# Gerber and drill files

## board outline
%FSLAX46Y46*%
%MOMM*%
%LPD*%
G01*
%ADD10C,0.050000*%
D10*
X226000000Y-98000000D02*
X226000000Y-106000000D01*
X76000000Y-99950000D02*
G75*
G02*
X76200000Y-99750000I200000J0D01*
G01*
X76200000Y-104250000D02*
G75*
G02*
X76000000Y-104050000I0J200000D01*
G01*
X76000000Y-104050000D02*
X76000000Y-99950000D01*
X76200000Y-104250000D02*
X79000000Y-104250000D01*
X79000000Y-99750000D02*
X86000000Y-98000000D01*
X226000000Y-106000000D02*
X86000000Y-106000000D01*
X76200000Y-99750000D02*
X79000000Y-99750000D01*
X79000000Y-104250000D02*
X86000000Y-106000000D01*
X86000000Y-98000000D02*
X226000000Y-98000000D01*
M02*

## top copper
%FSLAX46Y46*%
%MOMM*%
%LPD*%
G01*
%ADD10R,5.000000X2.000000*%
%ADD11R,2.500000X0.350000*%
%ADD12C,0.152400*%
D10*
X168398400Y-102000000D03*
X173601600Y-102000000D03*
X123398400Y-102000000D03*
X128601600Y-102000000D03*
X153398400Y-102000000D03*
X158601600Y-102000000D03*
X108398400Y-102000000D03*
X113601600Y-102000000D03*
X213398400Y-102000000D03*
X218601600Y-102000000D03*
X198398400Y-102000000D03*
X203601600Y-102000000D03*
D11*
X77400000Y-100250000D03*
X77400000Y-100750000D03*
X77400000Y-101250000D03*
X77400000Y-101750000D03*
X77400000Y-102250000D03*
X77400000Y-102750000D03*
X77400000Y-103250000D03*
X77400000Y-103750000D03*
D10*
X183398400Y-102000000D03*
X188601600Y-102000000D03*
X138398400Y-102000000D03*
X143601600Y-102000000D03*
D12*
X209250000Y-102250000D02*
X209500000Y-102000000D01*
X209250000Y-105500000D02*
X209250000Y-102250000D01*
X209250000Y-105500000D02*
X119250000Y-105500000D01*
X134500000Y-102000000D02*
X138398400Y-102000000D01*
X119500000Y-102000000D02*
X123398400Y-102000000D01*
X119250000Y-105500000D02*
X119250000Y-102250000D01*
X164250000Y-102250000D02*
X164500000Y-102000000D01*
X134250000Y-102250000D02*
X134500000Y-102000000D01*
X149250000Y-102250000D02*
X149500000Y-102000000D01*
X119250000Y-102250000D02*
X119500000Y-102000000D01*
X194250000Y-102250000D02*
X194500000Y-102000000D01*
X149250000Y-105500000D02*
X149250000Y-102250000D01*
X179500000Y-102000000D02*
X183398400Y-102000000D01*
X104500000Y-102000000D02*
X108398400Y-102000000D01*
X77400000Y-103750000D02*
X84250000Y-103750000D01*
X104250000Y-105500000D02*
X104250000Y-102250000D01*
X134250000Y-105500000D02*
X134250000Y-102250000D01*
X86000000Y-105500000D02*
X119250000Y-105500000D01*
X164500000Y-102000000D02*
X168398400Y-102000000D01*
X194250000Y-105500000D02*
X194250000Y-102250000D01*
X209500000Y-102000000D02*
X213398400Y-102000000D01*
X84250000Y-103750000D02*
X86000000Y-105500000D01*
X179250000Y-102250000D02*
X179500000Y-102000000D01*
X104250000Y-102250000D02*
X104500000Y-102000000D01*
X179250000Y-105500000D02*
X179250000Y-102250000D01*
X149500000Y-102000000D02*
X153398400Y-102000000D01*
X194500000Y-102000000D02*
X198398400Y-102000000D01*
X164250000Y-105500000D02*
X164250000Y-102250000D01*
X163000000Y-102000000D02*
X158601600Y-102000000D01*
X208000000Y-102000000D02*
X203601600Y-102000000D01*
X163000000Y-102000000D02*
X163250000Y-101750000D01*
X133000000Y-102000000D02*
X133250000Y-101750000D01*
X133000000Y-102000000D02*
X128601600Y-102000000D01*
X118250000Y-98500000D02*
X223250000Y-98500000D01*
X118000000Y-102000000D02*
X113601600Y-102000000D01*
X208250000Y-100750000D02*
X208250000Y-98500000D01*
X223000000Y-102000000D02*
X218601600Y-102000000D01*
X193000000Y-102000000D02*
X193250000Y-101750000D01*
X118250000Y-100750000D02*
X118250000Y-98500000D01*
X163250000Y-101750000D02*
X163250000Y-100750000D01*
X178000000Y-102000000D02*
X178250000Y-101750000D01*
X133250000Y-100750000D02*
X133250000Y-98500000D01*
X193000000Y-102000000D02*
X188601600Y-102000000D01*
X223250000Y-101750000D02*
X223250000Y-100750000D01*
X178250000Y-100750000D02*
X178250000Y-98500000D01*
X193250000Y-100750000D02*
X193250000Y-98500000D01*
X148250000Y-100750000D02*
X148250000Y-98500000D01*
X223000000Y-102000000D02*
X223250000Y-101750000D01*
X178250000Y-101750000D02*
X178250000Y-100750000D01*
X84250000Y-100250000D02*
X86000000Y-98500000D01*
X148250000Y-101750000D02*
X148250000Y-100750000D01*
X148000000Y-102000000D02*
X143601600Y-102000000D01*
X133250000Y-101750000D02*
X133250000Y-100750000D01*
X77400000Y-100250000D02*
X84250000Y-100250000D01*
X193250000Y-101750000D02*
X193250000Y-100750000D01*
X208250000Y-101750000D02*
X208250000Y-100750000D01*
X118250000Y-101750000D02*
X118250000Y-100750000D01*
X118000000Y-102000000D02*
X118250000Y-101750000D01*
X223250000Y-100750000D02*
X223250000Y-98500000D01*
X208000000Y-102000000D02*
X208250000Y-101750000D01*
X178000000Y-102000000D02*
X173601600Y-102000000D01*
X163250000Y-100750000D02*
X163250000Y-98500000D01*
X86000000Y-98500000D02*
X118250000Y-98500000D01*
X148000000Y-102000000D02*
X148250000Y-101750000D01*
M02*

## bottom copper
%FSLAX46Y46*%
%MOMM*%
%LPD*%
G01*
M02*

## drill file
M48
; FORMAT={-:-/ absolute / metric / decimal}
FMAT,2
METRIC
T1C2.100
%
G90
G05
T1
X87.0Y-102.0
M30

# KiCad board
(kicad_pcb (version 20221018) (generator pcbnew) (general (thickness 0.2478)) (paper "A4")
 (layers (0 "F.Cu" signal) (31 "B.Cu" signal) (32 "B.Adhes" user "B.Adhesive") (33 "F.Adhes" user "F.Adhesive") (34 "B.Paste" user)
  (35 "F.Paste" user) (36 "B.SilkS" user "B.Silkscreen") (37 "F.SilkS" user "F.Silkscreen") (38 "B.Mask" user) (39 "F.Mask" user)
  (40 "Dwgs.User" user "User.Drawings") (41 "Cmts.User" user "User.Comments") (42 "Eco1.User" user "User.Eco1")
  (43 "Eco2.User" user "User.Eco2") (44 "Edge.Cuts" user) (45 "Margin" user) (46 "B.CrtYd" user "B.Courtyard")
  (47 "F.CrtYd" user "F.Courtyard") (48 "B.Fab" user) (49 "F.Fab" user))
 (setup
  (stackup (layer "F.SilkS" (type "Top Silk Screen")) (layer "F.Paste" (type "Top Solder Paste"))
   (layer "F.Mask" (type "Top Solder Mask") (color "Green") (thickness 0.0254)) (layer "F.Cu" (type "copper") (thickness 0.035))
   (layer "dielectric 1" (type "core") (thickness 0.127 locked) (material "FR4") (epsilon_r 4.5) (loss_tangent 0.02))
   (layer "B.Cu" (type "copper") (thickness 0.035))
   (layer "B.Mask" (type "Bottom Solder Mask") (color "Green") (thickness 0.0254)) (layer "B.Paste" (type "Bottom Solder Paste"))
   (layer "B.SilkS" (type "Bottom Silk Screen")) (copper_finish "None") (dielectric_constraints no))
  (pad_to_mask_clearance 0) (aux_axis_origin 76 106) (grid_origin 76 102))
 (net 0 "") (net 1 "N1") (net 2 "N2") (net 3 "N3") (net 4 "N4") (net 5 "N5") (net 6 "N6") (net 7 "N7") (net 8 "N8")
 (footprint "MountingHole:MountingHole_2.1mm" (layer "F.Cu") (at 87 102)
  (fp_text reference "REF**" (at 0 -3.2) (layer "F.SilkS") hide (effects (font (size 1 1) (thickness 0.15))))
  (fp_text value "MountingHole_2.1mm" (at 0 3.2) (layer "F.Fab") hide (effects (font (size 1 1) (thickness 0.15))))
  (pad "" np_thru_hole circle (at 0 0) (size 2.1 2.1) (drill 2.1) (layers "*.Cu" "*.Mask")))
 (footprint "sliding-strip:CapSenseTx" (layer "F.Cu") (at 171 102)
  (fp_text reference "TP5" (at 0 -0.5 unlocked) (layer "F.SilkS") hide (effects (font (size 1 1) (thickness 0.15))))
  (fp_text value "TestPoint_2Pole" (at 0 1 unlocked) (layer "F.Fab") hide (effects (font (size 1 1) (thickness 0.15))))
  (pad "1" smd rect (at -2.6016 0) (size 5 2) (layers "F.Cu") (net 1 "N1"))
  (pad "2" smd rect (at 2.6016 0) (size 5 2) (layers "F.Cu") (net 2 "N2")))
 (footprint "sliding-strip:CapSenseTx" (layer "F.Cu") (at 126 102)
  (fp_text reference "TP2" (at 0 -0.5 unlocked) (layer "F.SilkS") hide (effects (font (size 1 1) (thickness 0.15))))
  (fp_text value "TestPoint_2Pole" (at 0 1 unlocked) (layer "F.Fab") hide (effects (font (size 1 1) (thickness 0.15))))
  (pad "1" smd rect (at -2.6016 0) (size 5 2) (layers "F.Cu") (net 1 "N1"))
  (pad "2" smd rect (at 2.6016 0) (size 5 2) (layers "F.Cu") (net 2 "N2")))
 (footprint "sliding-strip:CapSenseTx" (layer "F.Cu") (at 156 102)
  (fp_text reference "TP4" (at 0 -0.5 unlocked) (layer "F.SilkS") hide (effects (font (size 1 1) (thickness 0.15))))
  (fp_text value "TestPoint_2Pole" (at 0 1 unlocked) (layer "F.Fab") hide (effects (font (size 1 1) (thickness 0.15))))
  (pad "1" smd rect (at -2.6016 0) (size 5 2) (layers "F.Cu") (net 1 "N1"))
  (pad "2" smd rect (at 2.6016 0) (size 5 2) (layers "F.Cu") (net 2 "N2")))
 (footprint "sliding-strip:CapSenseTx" (layer "F.Cu") (at 111 102)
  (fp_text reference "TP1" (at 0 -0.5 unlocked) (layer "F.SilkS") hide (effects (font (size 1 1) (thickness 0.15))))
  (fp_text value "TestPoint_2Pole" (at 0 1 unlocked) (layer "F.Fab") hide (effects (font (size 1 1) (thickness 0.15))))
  (pad "1" smd rect (at -2.6016 0) (size 5 2) (layers "F.Cu") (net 1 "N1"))
  (pad "2" smd rect (at 2.6016 0) (size 5 2) (layers "F.Cu") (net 2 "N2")))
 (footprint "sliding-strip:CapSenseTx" (layer "F.Cu") (at 216 102)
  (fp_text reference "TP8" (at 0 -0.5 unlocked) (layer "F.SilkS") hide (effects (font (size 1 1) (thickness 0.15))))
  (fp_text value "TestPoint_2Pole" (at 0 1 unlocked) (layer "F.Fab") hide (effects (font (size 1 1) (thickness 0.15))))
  (pad "1" smd rect (at -2.6016 0) (size 5 2) (layers "F.Cu") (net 1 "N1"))
  (pad "2" smd rect (at 2.6016 0) (size 5 2) (layers "F.Cu") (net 2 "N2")))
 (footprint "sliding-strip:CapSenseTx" (layer "F.Cu") (at 201 102)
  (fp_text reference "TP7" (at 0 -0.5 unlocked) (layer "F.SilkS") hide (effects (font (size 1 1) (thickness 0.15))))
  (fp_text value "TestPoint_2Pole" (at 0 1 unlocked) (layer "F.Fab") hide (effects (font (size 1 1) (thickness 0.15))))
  (pad "1" smd rect (at -2.6016 0) (size 5 2) (layers "F.Cu") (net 1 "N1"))
  (pad "2" smd rect (at 2.6016 0) (size 5 2) (layers "F.Cu") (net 2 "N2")))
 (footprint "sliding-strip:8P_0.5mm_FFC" (layer "F.Cu") (at 77.4 102 -90)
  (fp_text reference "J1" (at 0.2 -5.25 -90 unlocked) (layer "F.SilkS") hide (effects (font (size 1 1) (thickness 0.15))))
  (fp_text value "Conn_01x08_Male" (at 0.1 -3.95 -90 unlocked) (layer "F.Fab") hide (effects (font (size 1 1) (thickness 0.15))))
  (pad "1" smd rect (at -1.75 0 270) (size 0.35 2.5) (layers "F.Cu" "F.Mask") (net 2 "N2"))
  (pad "2" smd rect (at -1.25 0 270) (size 0.35 2.5) (layers "F.Cu" "F.Mask") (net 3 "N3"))
  (pad "3" smd rect (at -0.75 0 270) (size 0.35 2.5) (layers "F.Cu" "F.Mask") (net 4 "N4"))
  (pad "4" smd rect (at -0.25 0 270) (size 0.35 2.5) (layers "F.Cu" "F.Mask") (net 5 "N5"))
  (pad "5" smd rect (at 0.25 0 270) (size 0.35 2.5) (layers "F.Cu" "F.Mask") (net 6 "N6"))
  (pad "6" smd rect (at 0.75 0 270) (size 0.35 2.5) (layers "F.Cu" "F.Mask") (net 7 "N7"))
  (pad "7" smd rect (at 1.25 0 270) (size 0.35 2.5) (layers "F.Cu" "F.Mask") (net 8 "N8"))
  (pad "8" smd rect (at 1.75 0 270) (size 0.35 2.5) (layers "F.Cu" "F.Mask") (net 1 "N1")))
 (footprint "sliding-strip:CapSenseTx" (layer "F.Cu") (at 186 102)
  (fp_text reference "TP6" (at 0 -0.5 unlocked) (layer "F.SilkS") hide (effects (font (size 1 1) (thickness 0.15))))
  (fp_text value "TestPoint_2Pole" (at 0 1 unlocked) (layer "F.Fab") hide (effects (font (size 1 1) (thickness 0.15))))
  (pad "1" smd rect (at -2.6016 0) (size 5 2) (layers "F.Cu") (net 1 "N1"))
  (pad "2" smd rect (at 2.6016 0) (size 5 2) (layers "F.Cu") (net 2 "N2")))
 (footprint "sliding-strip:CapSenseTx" (layer "F.Cu") (at 141 102)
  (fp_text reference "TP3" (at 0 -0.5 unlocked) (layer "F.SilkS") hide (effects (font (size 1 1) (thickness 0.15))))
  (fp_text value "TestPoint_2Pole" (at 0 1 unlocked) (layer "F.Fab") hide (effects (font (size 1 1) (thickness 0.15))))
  (pad "1" smd rect (at -2.6016 0) (size 5 2) (layers "F.Cu") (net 1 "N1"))
  (pad "2" smd rect (at 2.6016 0) (size 5 2) (layers "F.Cu") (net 2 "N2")))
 (gr_line (start 226 98) (end 226 106) (stroke (width 0.05) (type solid)) (layer "Edge.Cuts"))
 (gr_arc (start 76 99.95) (mid 76.058579 99.808579) (end 76.2 99.75) (stroke (width 0.05) (type solid)) (layer "Edge.Cuts"))
 (gr_arc (start 76.2 104.25) (mid 76.058579 104.191421) (end 76 104.05) (stroke (width 0.05) (type solid)) (layer "Edge.Cuts"))
 (gr_line (start 76 104.05) (end 76 99.95) (stroke (width 0.05) (type solid)) (layer "Edge.Cuts"))
 (gr_line (start 76.2 104.25) (end 79 104.25) (stroke (width 0.05) (type solid)) (layer "Edge.Cuts"))
 (gr_line (start 79 99.75) (end 86 98) (stroke (width 0.05) (type solid)) (layer "Edge.Cuts"))
 (gr_line (start 226 106) (end 86 106) (stroke (width 0.05) (type solid)) (layer "Edge.Cuts"))
 (gr_line (start 76.2 99.75) (end 79 99.75) (stroke (width 0.05) (type solid)) (layer "Edge.Cuts"))
 (gr_line (start 79 104.25) (end 86 106) (stroke (width 0.05) (type solid)) (layer "Edge.Cuts"))
 (gr_line (start 86 98) (end 226 98) (stroke (width 0.05) (type solid)) (layer "Edge.Cuts"))
 (segment (start 209.25 102.25) (end 209.5 102) (width 0.1524) (layer "F.Cu") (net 1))
 (segment (start 209.25 105.5) (end 209.25 102.25) (width 0.1524) (layer "F.Cu") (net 1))
 (segment (start 209.25 105.5) (end 119.25 105.5) (width 0.1524) (layer "F.Cu") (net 1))
 (segment (start 134.5 102) (end 138.3984 102) (width 0.1524) (layer "F.Cu") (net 1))
 (segment (start 119.5 102) (end 123.3984 102) (width 0.1524) (layer "F.Cu") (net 1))
 (segment (start 119.25 105.5) (end 119.25 102.25) (width 0.1524) (layer "F.Cu") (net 1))
 (segment (start 164.25 102.25) (end 164.5 102) (width 0.1524) (layer "F.Cu") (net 1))
 (segment (start 134.25 102.25) (end 134.5 102) (width 0.1524) (layer "F.Cu") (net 1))
 (segment (start 149.25 102.25) (end 149.5 102) (width 0.1524) (layer "F.Cu") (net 1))
 (segment (start 119.25 102.25) (end 119.5 102) (width 0.1524) (layer "F.Cu") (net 1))
 (segment (start 194.25 102.25) (end 194.5 102) (width 0.1524) (layer "F.Cu") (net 1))
 (segment (start 149.25 105.5) (end 149.25 102.25) (width 0.1524) (layer "F.Cu") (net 1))
 (segment (start 179.5 102) (end 183.3984 102) (width 0.1524) (layer "F.Cu") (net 1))
 (segment (start 104.5 102) (end 108.3984 102) (width 0.1524) (layer "F.Cu") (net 1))
 (segment (start 77.4 103.75) (end 84.25 103.75) (width 0.1524) (layer "F.Cu") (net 1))
 (segment (start 104.25 105.5) (end 104.25 102.25) (width 0.1524) (layer "F.Cu") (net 1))
 (segment (start 134.25 105.5) (end 134.25 102.25) (width 0.1524) (layer "F.Cu") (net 1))
 (segment (start 86 105.5) (end 119.25 105.5) (width 0.1524) (layer "F.Cu") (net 1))
 (segment (start 164.5 102) (end 168.3984 102) (width 0.1524) (layer "F.Cu") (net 1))
 (segment (start 194.25 105.5) (end 194.25 102.25) (width 0.1524) (layer "F.Cu") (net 1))
 (segment (start 209.5 102) (end 213.3984 102) (width 0.1524) (layer "F.Cu") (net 1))
 (segment (start 84.25 103.75) (end 86 105.5) (width 0.1524) (layer "F.Cu") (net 1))
 (segment (start 179.25 102.25) (end 179.5 102) (width 0.1524) (layer "F.Cu") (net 1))
 (segment (start 104.25 102.25) (end 104.5 102) (width 0.1524) (layer "F.Cu") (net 1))
 (segment (start 179.25 105.5) (end 179.25 102.25) (width 0.1524) (layer "F.Cu") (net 1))
 (segment (start 149.5 102) (end 153.3984 102) (width 0.1524) (layer "F.Cu") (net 1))
 (segment (start 194.5 102) (end 198.3984 102) (width 0.1524) (layer "F.Cu") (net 1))
 (segment (start 164.25 105.5) (end 164.25 102.25) (width 0.1524) (layer "F.Cu") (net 1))
 (segment (start 163 102) (end 158.6016 102) (width 0.1524) (layer "F.Cu") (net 2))
 (segment (start 208 102) (end 203.6016 102) (width 0.1524) (layer "F.Cu") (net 2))
 (segment (start 163 102) (end 163.25 101.75) (width 0.1524) (layer "F.Cu") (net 2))
 (segment (start 133 102) (end 133.25 101.75) (width 0.1524) (layer "F.Cu") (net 2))
 (segment (start 133 102) (end 128.6016 102) (width 0.1524) (layer "F.Cu") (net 2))
 (segment (start 118.25 98.5) (end 223.25 98.5) (width 0.1524) (layer "F.Cu") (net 2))
 (segment (start 118 102) (end 113.6016 102) (width 0.1524) (layer "F.Cu") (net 2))
 (segment (start 208.25 100.75) (end 208.25 98.5) (width 0.1524) (layer "F.Cu") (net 2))
 (segment (start 223 102) (end 218.6016 102) (width 0.1524) (layer "F.Cu") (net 2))
 (segment (start 193 102) (end 193.25 101.75) (width 0.1524) (layer "F.Cu") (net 2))
 (segment (start 118.25 100.75) (end 118.25 98.5) (width 0.1524) (layer "F.Cu") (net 2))
 (segment (start 163.25 101.75) (end 163.25 100.75) (width 0.1524) (layer "F.Cu") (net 2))
 (segment (start 178 102) (end 178.25 101.75) (width 0.1524) (layer "F.Cu") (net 2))
 (segment (start 133.25 100.75) (end 133.25 98.5) (width 0.1524) (layer "F.Cu") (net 2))
 (segment (start 193 102) (end 188.6016 102) (width 0.1524) (layer "F.Cu") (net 2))
 (segment (start 223.25 101.75) (end 223.25 100.75) (width 0.1524) (layer "F.Cu") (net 2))
 (segment (start 178.25 100.75) (end 178.25 98.5) (width 0.1524) (layer "F.Cu") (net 2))
 (segment (start 193.25 100.75) (end 193.25 98.5) (width 0.1524) (layer "F.Cu") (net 2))
 (segment (start 148.25 100.75) (end 148.25 98.5) (width 0.1524) (layer "F.Cu") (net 2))
 (segment (start 223 102) (end 223.25 101.75) (width 0.1524) (layer "F.Cu") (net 2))
 (segment (start 178.25 101.75) (end 178.25 100.75) (width 0.1524) (layer "F.Cu") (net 2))
 (segment (start 84.25 100.25) (end 86 98.5) (width 0.1524) (layer "F.Cu") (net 2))
 (segment (start 148.25 101.75) (end 148.25 100.75) (width 0.1524) (layer "F.Cu") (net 2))
 (segment (start 148 102) (end 143.6016 102) (width 0.1524) (layer "F.Cu") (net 2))
 (segment (start 133.25 101.75) (end 133.25 100.75) (width 0.1524) (layer "F.Cu") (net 2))
 (segment (start 77.4 100.25) (end 84.25 100.25) (width 0.1524) (layer "F.Cu") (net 2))
 (segment (start 193.25 101.75) (end 193.25 100.75) (width 0.1524) (layer "F.Cu") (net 2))
 (segment (start 208.25 101.75) (end 208.25 100.75) (width 0.1524) (layer "F.Cu") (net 2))
 (segment (start 118.25 101.75) (end 118.25 100.75) (width 0.1524) (layer "F.Cu") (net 2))
 (segment (start 118 102) (end 118.25 101.75) (width 0.1524) (layer "F.Cu") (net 2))
 (segment (start 223.25 100.75) (end 223.25 98.5) (width 0.1524) (layer "F.Cu") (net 2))
 (segment (start 208 102) (end 208.25 101.75) (width 0.1524) (layer "F.Cu") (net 2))
 (segment (start 178 102) (end 173.6016 102) (width 0.1524) (layer "F.Cu") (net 2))
 (segment (start 163.25 100.75) (end 163.25 98.5) (width 0.1524) (layer "F.Cu") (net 2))
 (segment (start 86 98.5) (end 118.25 98.5) (width 0.1524) (layer "F.Cu") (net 2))
 (segment (start 148 102) (end 148.25 101.75) (width 0.1524) (layer "F.Cu") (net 2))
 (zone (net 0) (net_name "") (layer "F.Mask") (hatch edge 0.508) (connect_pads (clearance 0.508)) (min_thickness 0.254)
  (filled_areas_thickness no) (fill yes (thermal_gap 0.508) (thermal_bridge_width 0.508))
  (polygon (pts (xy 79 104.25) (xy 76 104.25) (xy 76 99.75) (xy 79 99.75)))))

